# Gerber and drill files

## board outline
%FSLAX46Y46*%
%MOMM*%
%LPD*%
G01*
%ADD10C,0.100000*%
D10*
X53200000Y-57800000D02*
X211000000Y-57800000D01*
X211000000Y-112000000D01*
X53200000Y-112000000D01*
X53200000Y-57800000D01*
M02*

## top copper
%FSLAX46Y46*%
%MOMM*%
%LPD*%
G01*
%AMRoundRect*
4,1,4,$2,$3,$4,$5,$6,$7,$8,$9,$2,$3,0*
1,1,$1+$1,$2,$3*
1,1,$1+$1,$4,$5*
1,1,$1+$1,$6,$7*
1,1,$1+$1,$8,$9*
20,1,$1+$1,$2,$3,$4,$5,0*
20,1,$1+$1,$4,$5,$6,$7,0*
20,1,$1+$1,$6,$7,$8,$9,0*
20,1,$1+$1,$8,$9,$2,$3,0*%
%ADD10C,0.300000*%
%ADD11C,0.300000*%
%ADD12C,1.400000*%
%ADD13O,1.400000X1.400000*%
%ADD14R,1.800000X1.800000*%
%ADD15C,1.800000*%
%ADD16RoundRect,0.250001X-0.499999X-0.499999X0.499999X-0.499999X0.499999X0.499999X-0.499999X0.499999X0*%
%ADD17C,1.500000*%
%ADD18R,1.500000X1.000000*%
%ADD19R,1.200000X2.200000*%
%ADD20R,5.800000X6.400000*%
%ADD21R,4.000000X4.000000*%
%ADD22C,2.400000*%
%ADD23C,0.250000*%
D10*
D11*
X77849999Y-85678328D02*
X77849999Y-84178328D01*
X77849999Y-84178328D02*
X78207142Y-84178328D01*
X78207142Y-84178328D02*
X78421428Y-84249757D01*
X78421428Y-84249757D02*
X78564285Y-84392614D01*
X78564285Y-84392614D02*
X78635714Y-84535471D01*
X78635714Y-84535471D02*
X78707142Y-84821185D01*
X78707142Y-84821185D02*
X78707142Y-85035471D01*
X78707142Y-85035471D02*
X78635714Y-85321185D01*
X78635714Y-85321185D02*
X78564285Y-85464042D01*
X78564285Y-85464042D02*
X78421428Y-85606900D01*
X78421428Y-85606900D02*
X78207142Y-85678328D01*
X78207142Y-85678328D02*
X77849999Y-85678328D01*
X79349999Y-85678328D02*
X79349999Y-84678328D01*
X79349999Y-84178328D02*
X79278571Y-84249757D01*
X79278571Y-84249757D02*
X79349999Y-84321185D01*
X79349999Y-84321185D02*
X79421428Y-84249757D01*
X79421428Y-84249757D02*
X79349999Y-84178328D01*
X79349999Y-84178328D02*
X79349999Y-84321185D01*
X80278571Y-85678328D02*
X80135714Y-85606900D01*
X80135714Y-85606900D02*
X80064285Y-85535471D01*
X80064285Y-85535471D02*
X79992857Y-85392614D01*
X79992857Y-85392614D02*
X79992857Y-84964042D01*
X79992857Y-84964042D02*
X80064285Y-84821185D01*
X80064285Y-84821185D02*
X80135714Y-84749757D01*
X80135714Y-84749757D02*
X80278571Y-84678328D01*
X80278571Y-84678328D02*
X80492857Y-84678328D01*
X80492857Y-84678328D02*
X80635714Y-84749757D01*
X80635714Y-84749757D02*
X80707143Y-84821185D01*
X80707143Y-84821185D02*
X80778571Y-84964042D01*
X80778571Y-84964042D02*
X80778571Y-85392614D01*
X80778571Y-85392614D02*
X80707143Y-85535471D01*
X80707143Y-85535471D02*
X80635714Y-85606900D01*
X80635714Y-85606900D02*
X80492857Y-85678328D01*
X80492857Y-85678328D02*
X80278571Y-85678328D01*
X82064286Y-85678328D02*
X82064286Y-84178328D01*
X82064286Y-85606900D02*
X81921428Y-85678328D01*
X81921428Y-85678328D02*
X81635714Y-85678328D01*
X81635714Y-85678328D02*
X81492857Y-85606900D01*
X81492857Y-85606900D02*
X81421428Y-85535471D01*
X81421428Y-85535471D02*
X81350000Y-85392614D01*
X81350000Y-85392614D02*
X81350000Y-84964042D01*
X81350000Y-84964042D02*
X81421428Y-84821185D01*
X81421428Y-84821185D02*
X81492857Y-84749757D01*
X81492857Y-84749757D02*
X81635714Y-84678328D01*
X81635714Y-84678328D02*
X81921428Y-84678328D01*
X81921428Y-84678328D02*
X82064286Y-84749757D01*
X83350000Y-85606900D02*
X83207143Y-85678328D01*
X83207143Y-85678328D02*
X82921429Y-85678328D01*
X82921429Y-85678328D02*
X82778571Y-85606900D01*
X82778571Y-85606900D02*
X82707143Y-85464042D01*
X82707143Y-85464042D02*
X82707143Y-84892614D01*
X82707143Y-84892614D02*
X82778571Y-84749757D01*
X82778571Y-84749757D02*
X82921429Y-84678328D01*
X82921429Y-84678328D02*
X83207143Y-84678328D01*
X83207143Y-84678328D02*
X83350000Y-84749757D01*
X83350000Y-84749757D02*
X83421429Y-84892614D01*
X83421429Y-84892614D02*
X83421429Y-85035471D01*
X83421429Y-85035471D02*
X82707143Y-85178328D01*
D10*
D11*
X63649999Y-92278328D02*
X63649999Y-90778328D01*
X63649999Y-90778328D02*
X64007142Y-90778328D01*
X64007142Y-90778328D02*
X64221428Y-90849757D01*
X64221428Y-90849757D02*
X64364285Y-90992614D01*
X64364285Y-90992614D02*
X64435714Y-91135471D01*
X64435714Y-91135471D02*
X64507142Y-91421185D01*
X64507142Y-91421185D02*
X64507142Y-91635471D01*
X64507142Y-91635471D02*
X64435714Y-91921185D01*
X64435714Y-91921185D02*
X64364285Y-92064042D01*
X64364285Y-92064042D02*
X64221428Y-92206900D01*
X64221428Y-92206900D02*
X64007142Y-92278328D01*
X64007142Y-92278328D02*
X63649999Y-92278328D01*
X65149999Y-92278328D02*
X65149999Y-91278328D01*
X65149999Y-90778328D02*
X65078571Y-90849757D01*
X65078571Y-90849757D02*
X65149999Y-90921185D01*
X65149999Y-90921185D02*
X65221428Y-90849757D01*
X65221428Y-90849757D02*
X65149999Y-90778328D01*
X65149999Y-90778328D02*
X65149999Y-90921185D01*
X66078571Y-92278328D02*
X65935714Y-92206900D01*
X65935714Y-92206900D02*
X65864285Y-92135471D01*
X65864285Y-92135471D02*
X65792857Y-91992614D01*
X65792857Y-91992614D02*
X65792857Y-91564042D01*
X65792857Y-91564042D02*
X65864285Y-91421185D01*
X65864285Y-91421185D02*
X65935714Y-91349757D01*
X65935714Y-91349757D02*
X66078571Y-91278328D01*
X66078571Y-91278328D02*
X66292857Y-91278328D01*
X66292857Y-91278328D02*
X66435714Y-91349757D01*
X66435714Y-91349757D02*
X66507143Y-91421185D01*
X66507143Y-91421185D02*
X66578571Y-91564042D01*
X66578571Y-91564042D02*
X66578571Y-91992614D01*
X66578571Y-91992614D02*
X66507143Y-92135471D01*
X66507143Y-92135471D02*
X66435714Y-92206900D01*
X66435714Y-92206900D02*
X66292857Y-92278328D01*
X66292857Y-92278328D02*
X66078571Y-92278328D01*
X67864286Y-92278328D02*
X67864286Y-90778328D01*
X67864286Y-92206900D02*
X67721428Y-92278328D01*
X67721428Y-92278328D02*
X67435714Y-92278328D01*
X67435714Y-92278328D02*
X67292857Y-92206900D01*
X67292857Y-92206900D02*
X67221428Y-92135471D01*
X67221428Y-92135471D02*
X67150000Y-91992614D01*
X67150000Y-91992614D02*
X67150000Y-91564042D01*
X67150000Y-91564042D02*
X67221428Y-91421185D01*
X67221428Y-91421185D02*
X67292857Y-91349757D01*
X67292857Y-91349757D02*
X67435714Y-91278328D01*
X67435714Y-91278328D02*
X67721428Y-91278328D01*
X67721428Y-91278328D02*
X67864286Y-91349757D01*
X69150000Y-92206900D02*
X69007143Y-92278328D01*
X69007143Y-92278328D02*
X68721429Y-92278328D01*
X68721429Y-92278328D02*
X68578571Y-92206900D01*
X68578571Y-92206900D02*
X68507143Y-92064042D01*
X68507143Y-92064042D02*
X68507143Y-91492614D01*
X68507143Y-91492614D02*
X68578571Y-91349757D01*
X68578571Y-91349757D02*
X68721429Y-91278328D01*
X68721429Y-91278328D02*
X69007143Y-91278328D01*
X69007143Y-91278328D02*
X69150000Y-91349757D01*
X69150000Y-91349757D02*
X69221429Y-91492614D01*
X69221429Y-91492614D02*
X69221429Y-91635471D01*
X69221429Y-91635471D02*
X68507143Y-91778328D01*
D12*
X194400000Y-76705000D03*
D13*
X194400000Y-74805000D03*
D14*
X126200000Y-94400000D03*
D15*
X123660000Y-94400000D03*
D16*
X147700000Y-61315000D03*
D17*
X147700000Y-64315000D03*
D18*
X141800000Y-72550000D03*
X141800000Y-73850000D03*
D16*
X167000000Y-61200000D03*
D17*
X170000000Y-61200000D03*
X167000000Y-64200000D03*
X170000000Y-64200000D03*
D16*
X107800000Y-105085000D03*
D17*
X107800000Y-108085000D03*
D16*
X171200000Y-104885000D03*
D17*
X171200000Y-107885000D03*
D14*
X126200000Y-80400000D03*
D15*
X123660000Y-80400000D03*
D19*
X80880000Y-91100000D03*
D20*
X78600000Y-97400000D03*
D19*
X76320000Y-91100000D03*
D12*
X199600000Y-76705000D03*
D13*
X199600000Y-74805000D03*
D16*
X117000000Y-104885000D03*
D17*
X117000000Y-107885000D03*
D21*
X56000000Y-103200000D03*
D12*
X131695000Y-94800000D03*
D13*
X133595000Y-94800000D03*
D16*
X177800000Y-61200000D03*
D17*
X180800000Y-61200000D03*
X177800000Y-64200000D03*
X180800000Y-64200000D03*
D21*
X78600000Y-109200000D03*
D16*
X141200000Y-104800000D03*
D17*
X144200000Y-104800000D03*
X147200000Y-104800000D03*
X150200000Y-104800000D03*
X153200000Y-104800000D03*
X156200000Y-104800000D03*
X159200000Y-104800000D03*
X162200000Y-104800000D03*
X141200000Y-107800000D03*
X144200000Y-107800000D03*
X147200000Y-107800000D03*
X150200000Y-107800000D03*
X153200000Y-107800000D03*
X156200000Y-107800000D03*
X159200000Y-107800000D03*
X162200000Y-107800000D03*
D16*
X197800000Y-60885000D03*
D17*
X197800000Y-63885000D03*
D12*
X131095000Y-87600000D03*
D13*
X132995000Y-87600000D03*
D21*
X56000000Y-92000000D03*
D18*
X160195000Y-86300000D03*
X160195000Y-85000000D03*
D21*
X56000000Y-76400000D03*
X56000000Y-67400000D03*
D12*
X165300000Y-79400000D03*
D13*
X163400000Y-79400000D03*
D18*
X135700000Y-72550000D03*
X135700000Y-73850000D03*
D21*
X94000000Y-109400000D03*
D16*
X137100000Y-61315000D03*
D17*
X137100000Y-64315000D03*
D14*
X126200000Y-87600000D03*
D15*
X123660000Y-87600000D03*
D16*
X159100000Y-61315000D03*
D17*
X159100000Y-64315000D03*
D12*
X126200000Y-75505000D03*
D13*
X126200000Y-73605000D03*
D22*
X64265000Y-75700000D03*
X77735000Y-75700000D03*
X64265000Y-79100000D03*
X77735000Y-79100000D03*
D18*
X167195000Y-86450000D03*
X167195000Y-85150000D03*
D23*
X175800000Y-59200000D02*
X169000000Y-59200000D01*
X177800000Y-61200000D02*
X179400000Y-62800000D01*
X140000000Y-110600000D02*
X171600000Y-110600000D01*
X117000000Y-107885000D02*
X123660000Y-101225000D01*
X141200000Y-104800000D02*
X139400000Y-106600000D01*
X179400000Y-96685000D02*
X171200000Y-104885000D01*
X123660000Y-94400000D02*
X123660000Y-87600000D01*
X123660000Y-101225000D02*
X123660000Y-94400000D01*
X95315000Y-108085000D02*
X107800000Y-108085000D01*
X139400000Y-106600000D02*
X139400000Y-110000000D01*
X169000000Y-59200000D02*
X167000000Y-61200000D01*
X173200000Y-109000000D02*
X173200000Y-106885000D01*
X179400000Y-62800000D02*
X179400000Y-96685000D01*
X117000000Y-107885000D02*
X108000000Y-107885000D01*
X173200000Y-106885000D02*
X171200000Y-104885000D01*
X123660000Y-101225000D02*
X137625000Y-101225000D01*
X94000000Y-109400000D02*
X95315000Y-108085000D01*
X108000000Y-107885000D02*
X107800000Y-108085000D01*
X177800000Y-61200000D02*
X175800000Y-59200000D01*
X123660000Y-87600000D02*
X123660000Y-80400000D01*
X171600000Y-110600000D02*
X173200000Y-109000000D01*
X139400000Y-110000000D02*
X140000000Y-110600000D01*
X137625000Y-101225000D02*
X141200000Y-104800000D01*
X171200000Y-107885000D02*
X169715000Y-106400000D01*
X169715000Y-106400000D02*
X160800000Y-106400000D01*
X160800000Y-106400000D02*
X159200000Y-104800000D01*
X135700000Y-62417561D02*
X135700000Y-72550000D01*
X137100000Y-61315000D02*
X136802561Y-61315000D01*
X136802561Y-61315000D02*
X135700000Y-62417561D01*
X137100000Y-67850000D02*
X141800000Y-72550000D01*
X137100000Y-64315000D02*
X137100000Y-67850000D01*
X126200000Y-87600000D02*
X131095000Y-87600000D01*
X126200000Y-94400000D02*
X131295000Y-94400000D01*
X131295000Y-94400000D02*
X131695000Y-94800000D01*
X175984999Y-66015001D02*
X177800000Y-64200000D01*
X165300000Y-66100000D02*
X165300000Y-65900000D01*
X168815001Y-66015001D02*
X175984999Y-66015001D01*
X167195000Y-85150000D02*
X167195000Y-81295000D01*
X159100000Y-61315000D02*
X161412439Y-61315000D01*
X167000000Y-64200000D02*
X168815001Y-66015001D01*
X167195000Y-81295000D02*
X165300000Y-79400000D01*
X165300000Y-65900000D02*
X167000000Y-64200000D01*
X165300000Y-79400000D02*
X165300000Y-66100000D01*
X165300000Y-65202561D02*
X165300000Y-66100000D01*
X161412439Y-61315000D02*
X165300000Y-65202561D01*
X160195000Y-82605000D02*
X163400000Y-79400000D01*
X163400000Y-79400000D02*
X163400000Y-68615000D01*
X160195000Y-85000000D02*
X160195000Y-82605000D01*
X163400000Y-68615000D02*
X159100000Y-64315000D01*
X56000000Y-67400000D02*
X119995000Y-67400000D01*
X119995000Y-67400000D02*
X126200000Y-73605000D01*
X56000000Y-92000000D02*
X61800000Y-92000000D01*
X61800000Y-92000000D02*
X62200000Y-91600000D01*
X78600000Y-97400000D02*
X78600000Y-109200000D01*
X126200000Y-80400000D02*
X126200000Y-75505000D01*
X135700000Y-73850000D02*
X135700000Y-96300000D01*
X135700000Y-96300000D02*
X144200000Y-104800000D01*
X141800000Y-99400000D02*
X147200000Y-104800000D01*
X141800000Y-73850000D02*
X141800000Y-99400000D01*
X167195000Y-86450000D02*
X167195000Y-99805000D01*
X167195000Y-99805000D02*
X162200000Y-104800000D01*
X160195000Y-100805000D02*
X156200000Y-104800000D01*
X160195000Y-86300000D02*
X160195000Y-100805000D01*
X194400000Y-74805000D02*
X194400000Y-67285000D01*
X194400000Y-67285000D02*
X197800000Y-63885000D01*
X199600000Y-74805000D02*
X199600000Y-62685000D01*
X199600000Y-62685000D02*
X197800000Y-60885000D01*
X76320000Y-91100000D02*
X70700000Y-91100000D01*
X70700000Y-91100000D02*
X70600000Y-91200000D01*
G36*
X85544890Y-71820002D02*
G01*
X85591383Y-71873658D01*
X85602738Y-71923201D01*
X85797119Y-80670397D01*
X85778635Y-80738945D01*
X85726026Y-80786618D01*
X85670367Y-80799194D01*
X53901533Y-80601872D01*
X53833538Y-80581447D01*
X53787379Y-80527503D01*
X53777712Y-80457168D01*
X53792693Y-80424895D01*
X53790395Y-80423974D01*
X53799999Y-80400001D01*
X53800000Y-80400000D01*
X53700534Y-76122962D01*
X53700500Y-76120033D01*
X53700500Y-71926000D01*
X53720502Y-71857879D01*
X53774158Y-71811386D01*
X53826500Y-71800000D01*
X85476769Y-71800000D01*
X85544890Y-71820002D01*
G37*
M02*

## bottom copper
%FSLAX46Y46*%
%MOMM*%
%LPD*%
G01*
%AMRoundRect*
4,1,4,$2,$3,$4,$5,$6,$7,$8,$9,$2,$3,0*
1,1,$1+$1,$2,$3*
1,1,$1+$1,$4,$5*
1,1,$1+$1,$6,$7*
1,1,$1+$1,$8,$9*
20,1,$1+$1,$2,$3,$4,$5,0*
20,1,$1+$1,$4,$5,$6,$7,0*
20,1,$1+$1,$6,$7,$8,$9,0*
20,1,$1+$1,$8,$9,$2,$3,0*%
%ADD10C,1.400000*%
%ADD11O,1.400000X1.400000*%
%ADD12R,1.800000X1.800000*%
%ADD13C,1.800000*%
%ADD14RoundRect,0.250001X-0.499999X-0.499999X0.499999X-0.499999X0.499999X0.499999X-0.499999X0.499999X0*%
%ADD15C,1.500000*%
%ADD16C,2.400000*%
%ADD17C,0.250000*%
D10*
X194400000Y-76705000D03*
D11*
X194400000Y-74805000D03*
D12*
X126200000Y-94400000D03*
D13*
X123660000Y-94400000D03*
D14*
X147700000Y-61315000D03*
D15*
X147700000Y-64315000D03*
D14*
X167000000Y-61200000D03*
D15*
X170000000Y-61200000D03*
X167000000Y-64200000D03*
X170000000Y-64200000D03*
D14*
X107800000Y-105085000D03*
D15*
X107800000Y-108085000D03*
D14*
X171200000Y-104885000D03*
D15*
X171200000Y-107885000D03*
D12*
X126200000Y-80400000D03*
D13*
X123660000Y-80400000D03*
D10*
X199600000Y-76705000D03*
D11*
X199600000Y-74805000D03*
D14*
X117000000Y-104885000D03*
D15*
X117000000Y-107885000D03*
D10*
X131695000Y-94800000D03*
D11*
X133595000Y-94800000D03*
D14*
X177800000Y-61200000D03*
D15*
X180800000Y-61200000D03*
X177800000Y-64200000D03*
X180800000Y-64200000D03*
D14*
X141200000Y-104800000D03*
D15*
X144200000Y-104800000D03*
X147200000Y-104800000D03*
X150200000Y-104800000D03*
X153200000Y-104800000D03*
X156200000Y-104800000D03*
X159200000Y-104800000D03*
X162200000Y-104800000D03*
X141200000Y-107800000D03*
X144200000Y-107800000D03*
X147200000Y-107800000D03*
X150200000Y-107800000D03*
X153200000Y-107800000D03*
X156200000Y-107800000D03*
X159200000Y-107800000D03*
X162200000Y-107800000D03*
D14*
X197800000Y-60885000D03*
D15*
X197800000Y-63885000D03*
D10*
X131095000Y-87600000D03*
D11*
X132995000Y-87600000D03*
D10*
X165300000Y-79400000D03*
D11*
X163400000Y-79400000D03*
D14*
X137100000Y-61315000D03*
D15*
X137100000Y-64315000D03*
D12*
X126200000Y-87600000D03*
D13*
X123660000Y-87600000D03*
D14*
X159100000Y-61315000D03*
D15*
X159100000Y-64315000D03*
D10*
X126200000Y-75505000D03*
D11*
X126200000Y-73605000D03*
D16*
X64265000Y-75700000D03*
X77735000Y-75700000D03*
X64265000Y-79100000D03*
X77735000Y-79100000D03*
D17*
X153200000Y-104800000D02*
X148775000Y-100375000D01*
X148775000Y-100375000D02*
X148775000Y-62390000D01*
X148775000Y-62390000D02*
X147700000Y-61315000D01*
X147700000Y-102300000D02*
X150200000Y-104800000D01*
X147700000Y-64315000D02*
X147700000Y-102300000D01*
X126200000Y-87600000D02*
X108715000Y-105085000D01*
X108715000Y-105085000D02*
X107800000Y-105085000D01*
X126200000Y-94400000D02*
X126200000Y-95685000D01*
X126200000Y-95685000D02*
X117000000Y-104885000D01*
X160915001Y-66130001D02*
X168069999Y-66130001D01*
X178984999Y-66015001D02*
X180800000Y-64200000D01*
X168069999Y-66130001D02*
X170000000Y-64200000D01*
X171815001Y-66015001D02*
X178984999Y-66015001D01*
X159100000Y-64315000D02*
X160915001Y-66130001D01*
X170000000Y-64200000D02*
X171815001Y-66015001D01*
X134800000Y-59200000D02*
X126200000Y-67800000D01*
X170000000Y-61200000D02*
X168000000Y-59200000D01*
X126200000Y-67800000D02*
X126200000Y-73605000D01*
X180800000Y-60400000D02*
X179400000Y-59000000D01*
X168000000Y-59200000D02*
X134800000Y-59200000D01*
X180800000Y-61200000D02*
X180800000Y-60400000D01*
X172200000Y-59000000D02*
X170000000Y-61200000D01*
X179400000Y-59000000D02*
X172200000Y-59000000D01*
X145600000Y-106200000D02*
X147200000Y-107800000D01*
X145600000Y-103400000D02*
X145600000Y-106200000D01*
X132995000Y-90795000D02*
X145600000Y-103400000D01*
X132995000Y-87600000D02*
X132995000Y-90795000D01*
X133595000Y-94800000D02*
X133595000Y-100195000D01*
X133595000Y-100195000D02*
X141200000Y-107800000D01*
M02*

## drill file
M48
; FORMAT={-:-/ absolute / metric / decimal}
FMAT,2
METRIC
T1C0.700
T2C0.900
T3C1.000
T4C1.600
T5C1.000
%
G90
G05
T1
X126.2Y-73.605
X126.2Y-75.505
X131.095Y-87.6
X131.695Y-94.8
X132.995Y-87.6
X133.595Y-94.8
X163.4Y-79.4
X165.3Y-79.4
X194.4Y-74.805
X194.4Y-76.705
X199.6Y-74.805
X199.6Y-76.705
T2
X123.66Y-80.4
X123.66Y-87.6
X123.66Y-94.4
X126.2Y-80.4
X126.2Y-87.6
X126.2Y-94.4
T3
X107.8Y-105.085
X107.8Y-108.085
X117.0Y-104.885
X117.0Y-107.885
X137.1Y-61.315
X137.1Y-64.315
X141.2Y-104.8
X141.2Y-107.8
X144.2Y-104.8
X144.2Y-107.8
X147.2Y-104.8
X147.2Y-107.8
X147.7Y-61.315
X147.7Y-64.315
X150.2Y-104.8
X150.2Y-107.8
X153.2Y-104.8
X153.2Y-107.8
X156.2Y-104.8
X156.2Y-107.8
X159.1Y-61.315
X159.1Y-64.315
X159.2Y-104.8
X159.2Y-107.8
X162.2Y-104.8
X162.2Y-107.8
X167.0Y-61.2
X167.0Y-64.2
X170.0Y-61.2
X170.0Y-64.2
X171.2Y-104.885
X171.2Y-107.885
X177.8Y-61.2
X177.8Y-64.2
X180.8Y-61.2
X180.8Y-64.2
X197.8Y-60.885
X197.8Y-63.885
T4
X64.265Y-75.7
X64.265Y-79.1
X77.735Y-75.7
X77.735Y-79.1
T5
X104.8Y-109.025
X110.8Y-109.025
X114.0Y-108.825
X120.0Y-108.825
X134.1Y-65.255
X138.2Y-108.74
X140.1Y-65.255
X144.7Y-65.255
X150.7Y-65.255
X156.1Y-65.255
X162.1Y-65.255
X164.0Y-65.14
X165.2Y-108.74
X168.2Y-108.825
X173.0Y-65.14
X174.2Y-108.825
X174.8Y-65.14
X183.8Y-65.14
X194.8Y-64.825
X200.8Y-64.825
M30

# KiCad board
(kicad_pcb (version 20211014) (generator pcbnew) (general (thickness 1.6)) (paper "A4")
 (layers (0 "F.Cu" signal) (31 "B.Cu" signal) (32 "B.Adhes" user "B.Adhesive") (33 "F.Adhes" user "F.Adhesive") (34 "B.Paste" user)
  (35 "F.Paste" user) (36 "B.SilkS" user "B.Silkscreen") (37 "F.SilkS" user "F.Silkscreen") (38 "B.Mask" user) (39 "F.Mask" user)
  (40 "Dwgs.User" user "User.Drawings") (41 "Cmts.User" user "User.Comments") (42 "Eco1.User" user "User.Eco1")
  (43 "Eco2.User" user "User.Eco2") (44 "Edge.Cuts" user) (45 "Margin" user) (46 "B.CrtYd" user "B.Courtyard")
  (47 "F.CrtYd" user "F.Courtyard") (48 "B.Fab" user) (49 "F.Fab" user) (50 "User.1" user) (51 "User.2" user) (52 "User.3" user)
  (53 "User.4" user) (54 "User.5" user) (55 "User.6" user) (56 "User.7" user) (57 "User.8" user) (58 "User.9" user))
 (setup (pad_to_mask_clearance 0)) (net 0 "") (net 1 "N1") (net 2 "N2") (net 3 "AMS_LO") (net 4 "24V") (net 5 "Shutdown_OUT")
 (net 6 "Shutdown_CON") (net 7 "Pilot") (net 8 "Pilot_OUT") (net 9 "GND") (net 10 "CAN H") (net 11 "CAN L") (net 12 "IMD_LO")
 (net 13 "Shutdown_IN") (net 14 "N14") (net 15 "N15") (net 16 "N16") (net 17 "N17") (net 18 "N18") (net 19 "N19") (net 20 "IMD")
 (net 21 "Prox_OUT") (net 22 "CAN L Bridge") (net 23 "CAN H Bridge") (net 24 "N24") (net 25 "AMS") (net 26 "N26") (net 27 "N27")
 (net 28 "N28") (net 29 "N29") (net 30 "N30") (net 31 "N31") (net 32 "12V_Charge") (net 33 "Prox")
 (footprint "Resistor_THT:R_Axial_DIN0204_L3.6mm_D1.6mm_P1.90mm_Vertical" (layer "F.Cu") (at 194.4 76.705 90)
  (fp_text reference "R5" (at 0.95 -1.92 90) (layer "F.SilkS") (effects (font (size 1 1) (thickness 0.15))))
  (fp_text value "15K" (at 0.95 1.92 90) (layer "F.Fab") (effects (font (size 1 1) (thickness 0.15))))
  (pad "1" thru_hole circle (at 0 0 90) (size 1.4 1.4) (drill 0.7) (layers *.Cu *.Mask) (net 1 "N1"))
  (pad "2" thru_hole oval (at 1.9 0 90) (size 1.4 1.4) (drill 0.7) (layers *.Cu *.Mask) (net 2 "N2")))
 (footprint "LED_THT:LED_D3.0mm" (layer "F.Cu") (at 126.2 94.4 180)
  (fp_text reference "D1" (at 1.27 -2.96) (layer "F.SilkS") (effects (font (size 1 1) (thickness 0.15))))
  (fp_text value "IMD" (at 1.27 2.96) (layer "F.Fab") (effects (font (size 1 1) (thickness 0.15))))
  (pad "1" thru_hole rect (at 0 0 180) (size 1.8 1.8) (drill 0.9) (layers *.Cu *.Mask) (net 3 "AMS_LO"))
  (pad "2" thru_hole circle (at 2.54 0 180) (size 1.8 1.8) (drill 0.9) (layers *.Cu *.Mask) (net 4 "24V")))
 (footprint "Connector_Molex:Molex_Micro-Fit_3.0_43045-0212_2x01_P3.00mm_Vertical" (layer "F.Cu") (at 147.7 61.315)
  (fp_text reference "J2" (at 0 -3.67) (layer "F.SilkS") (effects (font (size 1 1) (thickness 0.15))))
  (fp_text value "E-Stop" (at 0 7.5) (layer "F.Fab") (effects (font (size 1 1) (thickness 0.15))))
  (pad "" np_thru_hole circle (at -3 3.94) (size 1 1) (drill 1) (layers *.Cu *.Mask))
  (pad "" np_thru_hole circle (at 3 3.94) (size 1 1) (drill 1) (layers *.Cu *.Mask))
  (pad "1" thru_hole roundrect (at 0 0) (size 1.5 1.5) (drill 1) (layers *.Cu *.Mask) (roundrect_rratio 0.166667) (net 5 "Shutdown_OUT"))
  (pad "2" thru_hole circle (at 0 3) (size 1.5 1.5) (drill 1) (layers *.Cu *.Mask) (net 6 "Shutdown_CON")))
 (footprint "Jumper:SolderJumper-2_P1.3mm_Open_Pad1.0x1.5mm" (layer "F.Cu") (at 141.8 73.2 -90)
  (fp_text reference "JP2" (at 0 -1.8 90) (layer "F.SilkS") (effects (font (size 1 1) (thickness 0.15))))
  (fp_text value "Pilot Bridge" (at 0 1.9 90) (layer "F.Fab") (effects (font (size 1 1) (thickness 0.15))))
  (pad "1" smd rect (at -0.65 0 270) (size 1 1.5) (layers "F.Cu" "F.Mask") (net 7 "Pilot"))
  (pad "2" smd rect (at 0.65 0 270) (size 1 1.5) (layers "F.Cu" "F.Mask") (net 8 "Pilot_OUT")))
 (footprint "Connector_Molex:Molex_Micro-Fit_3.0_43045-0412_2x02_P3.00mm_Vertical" (layer "F.Cu") (at 167 61.2)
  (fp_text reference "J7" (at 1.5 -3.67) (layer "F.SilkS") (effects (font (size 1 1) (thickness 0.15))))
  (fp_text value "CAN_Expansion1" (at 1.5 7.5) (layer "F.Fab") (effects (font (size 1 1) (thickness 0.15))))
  (pad "" np_thru_hole circle (at -3 3.94) (size 1 1) (drill 1) (layers *.Cu *.Mask))
  (pad "" np_thru_hole circle (at 6 3.94) (size 1 1) (drill 1) (layers *.Cu *.Mask))
  (pad "1" thru_hole roundrect (at 0 0) (size 1.5 1.5) (drill 1) (layers *.Cu *.Mask) (roundrect_rratio 0.166667) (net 4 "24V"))
  (pad "2" thru_hole circle (at 3 0) (size 1.5 1.5) (drill 1) (layers *.Cu *.Mask) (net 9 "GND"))
  (pad "3" thru_hole circle (at 0 3) (size 1.5 1.5) (drill 1) (layers *.Cu *.Mask) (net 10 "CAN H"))
  (pad "4" thru_hole circle (at 3 3) (size 1.5 1.5) (drill 1) (layers *.Cu *.Mask) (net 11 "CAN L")))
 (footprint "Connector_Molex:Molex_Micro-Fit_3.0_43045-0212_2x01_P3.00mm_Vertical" (layer "F.Cu") (at 107.8 105.085)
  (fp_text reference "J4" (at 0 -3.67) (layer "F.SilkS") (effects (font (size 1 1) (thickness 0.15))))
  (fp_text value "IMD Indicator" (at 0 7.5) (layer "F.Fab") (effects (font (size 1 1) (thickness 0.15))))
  (pad "" np_thru_hole circle (at -3 3.94) (size 1 1) (drill 1) (layers *.Cu *.Mask))
  (pad "" np_thru_hole circle (at 3 3.94) (size 1 1) (drill 1) (layers *.Cu *.Mask))
  (pad "1" thru_hole roundrect (at 0 0) (size 1.5 1.5) (drill 1) (layers *.Cu *.Mask) (roundrect_rratio 0.166667) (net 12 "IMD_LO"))
  (pad "2" thru_hole circle (at 0 3) (size 1.5 1.5) (drill 1) (layers *.Cu *.Mask) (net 4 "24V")))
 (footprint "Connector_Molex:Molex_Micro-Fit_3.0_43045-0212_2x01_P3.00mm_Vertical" (layer "F.Cu") (at 171.2 104.885)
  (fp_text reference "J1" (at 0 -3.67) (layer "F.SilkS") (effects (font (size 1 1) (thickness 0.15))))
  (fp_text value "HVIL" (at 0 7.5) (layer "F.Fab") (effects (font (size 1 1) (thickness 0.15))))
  (pad "" np_thru_hole circle (at -3 3.94) (size 1 1) (drill 1) (layers *.Cu *.Mask))
  (pad "" np_thru_hole circle (at 3 3.94) (size 1 1) (drill 1) (layers *.Cu *.Mask))
  (pad "1" thru_hole roundrect (at 0 0) (size 1.5 1.5) (drill 1) (layers *.Cu *.Mask) (roundrect_rratio 0.166667) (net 4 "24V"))
  (pad "2" thru_hole circle (at 0 3) (size 1.5 1.5) (drill 1) (layers *.Cu *.Mask) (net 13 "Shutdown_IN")))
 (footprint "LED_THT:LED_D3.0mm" (layer "F.Cu") (at 126.2 80.4 180)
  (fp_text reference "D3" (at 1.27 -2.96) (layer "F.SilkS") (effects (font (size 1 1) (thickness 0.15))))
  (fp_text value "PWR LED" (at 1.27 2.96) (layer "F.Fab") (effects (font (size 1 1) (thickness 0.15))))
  (pad "1" thru_hole rect (at 0 0 180) (size 1.8 1.8) (drill 0.9) (layers *.Cu *.Mask) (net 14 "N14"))
  (pad "2" thru_hole circle (at 2.54 0 180) (size 1.8 1.8) (drill 0.9) (layers *.Cu *.Mask) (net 4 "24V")))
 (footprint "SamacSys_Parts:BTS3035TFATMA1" (layer "F.Cu") (at 78.6 100.6 180)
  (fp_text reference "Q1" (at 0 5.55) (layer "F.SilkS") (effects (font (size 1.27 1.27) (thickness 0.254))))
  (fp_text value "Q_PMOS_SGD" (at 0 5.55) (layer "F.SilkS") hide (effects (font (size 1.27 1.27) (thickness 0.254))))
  (pad "1" smd rect locked (at -2.28 9.5 180) (size 1.2 2.2) (layers "F.Cu" "F.Paste" "F.Mask") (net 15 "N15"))
  (pad "2" smd rect locked (at 0 3.2 180) (size 5.8 6.4) (layers "F.Cu" "F.Paste" "F.Mask") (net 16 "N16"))
  (pad "3" smd rect locked (at 2.28 9.5 180) (size 1.2 2.2) (layers "F.Cu" "F.Paste" "F.Mask") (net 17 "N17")))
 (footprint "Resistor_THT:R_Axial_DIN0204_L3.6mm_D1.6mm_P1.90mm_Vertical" (layer "F.Cu") (at 199.6 76.705 90)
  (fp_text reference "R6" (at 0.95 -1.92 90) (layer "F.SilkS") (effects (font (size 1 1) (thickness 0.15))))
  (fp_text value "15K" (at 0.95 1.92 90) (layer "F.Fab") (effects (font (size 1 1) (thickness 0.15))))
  (pad "1" thru_hole circle (at 0 0 90) (size 1.4 1.4) (drill 0.7) (layers *.Cu *.Mask) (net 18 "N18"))
  (pad "2" thru_hole oval (at 1.9 0 90) (size 1.4 1.4) (drill 0.7) (layers *.Cu *.Mask) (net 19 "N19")))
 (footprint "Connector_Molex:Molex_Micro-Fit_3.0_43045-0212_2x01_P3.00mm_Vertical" (layer "F.Cu") (at 117 104.885)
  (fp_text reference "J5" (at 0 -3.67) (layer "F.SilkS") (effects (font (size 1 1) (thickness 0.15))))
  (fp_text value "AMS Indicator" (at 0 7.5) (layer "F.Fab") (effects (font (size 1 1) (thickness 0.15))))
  (pad "" np_thru_hole circle (at 3 3.94) (size 1 1) (drill 1) (layers *.Cu *.Mask))
  (pad "" np_thru_hole circle (at -3 3.94) (size 1 1) (drill 1) (layers *.Cu *.Mask))
  (pad "1" thru_hole roundrect (at 0 0) (size 1.5 1.5) (drill 1) (layers *.Cu *.Mask) (roundrect_rratio 0.166667) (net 3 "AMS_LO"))
  (pad "2" thru_hole circle (at 0 3) (size 1.5 1.5) (drill 1) (layers *.Cu *.Mask) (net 4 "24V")))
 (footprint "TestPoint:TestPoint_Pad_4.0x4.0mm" (layer "F.Cu") (at 56 103.2)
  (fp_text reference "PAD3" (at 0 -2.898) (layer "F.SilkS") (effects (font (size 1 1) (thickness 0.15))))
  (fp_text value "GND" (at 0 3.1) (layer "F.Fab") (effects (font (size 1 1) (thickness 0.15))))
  (pad "1" smd rect (at 0 0) (size 4 4) (layers "F.Cu" "F.Mask") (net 9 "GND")))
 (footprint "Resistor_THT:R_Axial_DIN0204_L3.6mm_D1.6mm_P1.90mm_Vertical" (layer "F.Cu") (at 131.695 94.8)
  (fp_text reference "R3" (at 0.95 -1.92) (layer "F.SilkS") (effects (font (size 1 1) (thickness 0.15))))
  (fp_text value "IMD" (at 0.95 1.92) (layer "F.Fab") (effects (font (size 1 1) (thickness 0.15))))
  (pad "1" thru_hole circle (at 0 0) (size 1.4 1.4) (drill 0.7) (layers *.Cu *.Mask) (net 3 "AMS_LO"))
  (pad "2" thru_hole oval (at 1.9 0) (size 1.4 1.4) (drill 0.7) (layers *.Cu *.Mask) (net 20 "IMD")))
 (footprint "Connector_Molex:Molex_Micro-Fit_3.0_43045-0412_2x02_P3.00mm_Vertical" (layer "F.Cu") (at 177.8 61.2)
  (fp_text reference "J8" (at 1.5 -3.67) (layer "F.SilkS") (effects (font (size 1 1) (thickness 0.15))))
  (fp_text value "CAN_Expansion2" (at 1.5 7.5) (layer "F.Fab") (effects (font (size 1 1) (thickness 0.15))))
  (pad "" np_thru_hole circle (at 6 3.94) (size 1 1) (drill 1) (layers *.Cu *.Mask))
  (pad "" np_thru_hole circle (at -3 3.94) (size 1 1) (drill 1) (layers *.Cu *.Mask))
  (pad "1" thru_hole roundrect (at 0 0) (size 1.5 1.5) (drill 1) (layers *.Cu *.Mask) (roundrect_rratio 0.166667) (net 4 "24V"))
  (pad "2" thru_hole circle (at 3 0) (size 1.5 1.5) (drill 1) (layers *.Cu *.Mask) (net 9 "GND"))
  (pad "3" thru_hole circle (at 0 3) (size 1.5 1.5) (drill 1) (layers *.Cu *.Mask) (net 10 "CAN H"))
  (pad "4" thru_hole circle (at 3 3) (size 1.5 1.5) (drill 1) (layers *.Cu *.Mask) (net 11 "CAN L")))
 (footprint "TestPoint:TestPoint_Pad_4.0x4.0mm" (layer "F.Cu") (at 78.6 109.2)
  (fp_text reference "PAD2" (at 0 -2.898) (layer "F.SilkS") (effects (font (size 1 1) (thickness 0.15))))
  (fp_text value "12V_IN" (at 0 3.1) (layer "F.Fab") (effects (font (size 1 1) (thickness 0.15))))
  (pad "1" smd rect (at 0 0) (size 4 4) (layers "F.Cu" "F.Mask") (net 16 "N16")))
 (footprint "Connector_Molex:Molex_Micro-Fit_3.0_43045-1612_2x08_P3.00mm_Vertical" (layer "F.Cu") (at 141.2 104.8)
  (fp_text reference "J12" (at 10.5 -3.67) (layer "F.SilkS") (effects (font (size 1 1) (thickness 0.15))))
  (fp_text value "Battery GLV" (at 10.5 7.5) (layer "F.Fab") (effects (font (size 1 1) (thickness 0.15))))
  (pad "" np_thru_hole circle (at -3 3.94) (size 1 1) (drill 1) (layers *.Cu *.Mask))
  (pad "" np_thru_hole circle (at 24 3.94) (size 1 1) (drill 1) (layers *.Cu *.Mask))
  (pad "1" thru_hole roundrect (at 0 0) (size 1.5 1.5) (drill 1) (layers *.Cu *.Mask) (roundrect_rratio 0.166667) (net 4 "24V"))
  (pad "2" thru_hole circle (at 3 0) (size 1.5 1.5) (drill 1) (layers *.Cu *.Mask) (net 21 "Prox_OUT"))
  (pad "3" thru_hole circle (at 6 0) (size 1.5 1.5) (drill 1) (layers *.Cu *.Mask) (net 8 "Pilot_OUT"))
  (pad "4" thru_hole circle (at 9 0) (size 1.5 1.5) (drill 1) (layers *.Cu *.Mask) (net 6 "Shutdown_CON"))
  (pad "5" thru_hole circle (at 12 0) (size 1.5 1.5) (drill 1) (layers *.Cu *.Mask) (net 5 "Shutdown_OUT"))
  (pad "6" thru_hole circle (at 15 0) (size 1.5 1.5) (drill 1) (layers *.Cu *.Mask) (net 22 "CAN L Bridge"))
  (pad "7" thru_hole circle (at 18 0) (size 1.5 1.5) (drill 1) (layers *.Cu *.Mask) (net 13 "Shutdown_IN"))
  (pad "8" thru_hole circle (at 21 0) (size 1.5 1.5) (drill 1) (layers *.Cu *.Mask) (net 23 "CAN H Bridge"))
  (pad "9" thru_hole circle (at 0 3) (size 1.5 1.5) (drill 1) (layers *.Cu *.Mask) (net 20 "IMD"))
  (pad "10" thru_hole circle (at 3 3) (size 1.5 1.5) (drill 1) (layers *.Cu *.Mask) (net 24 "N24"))
  (pad "11" thru_hole circle (at 6 3) (size 1.5 1.5) (drill 1) (layers *.Cu *.Mask) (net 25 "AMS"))
  (pad "12" thru_hole circle (at 9 3) (size 1.5 1.5) (drill 1) (layers *.Cu *.Mask) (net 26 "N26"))
  (pad "13" thru_hole circle (at 12 3) (size 1.5 1.5) (drill 1) (layers *.Cu *.Mask) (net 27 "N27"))
  (pad "14" thru_hole circle (at 15 3) (size 1.5 1.5) (drill 1) (layers *.Cu *.Mask) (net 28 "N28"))
  (pad "15" thru_hole circle (at 18 3) (size 1.5 1.5) (drill 1) (layers *.Cu *.Mask) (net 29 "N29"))
  (pad "16" thru_hole circle (at 21 3) (size 1.5 1.5) (drill 1) (layers *.Cu *.Mask) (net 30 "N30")))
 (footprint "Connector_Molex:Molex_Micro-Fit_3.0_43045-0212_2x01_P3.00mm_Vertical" (layer "F.Cu") (at 197.8 60.885)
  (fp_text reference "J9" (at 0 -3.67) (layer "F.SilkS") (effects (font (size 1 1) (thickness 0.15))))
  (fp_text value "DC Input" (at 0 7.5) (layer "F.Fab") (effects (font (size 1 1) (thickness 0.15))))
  (pad "" np_thru_hole circle (at -3 3.94) (size 1 1) (drill 1) (layers *.Cu *.Mask))
  (pad "" np_thru_hole circle (at 3 3.94) (size 1 1) (drill 1) (layers *.Cu *.Mask))
  (pad "1" thru_hole roundrect (at 0 0) (size 1.5 1.5) (drill 1) (layers *.Cu *.Mask) (roundrect_rratio 0.166667) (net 19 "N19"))
  (pad "2" thru_hole circle (at 0 3) (size 1.5 1.5) (drill 1) (layers *.Cu *.Mask) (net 2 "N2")))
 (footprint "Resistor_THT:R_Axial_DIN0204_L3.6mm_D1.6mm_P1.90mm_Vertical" (layer "F.Cu") (at 131.095 87.6)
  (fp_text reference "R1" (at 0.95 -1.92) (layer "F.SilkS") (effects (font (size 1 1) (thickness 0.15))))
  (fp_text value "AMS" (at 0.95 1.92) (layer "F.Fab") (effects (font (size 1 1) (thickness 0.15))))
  (pad "1" thru_hole circle (at 0 0) (size 1.4 1.4) (drill 0.7) (layers *.Cu *.Mask) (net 12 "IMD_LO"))
  (pad "2" thru_hole oval (at 1.9 0) (size 1.4 1.4) (drill 0.7) (layers *.Cu *.Mask) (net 25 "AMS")))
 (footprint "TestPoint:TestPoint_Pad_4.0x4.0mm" (layer "F.Cu") (at 56 92)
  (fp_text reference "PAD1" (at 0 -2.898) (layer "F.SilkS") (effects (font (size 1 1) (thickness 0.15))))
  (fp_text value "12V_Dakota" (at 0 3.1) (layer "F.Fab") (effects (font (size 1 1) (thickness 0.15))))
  (pad "1" smd rect (at 0 0) (size 4 4) (layers "F.Cu" "F.Mask") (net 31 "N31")))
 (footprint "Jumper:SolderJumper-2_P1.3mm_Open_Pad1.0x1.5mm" (layer "F.Cu") (at 160.195 85.65 90)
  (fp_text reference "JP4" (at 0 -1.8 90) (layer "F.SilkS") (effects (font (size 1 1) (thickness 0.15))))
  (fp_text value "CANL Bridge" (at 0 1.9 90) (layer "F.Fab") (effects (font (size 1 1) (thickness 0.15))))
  (pad "1" smd rect (at -0.65 0 90) (size 1 1.5) (layers "F.Cu" "F.Mask") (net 22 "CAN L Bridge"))
  (pad "2" smd rect (at 0.65 0 90) (size 1 1.5) (layers "F.Cu" "F.Mask") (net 11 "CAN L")))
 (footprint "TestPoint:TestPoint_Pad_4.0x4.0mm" (layer "F.Cu") (at 56 76.4)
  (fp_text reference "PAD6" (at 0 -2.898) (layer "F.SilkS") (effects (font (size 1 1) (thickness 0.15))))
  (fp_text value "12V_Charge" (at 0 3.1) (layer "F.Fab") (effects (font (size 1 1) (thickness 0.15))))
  (pad "1" smd rect (at 0 0) (size 4 4) (layers "F.Cu" "F.Mask") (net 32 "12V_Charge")))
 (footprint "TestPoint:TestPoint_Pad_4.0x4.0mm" (layer "F.Cu") (at 56 67.4)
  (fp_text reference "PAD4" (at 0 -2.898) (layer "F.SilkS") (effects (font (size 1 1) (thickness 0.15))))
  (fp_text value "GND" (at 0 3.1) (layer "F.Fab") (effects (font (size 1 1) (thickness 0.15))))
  (pad "1" smd rect (at 0 0) (size 4 4) (layers "F.Cu" "F.Mask") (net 9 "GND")))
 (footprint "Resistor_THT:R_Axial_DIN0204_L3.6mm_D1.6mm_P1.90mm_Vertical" (layer "F.Cu") (at 165.3 79.4 180)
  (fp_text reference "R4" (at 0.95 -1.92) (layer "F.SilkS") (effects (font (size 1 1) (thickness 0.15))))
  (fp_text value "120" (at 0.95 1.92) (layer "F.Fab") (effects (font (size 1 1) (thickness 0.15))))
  (pad "1" thru_hole circle (at 0 0 180) (size 1.4 1.4) (drill 0.7) (layers *.Cu *.Mask) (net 10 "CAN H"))
  (pad "2" thru_hole oval (at 1.9 0 180) (size 1.4 1.4) (drill 0.7) (layers *.Cu *.Mask) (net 11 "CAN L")))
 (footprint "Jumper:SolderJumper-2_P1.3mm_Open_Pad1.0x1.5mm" (layer "F.Cu") (at 135.7 73.2 -90)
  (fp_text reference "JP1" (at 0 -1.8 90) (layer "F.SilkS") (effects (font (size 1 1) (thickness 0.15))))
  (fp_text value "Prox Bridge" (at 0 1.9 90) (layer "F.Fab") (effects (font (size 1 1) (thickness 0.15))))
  (pad "1" smd rect (at -0.65 0 270) (size 1 1.5) (layers "F.Cu" "F.Mask") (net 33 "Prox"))
  (pad "2" smd rect (at 0.65 0 270) (size 1 1.5) (layers "F.Cu" "F.Mask") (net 21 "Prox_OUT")))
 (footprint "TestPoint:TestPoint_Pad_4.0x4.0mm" (layer "F.Cu") (at 94 109.4)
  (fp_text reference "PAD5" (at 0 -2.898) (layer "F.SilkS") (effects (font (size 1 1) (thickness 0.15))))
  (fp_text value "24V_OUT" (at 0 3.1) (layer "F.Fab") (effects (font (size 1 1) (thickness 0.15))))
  (pad "1" smd rect (at 0 0) (size 4 4) (layers "F.Cu" "F.Mask") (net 4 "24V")))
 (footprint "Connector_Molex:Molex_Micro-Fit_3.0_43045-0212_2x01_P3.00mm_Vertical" (layer "F.Cu") (at 137.1 61.315)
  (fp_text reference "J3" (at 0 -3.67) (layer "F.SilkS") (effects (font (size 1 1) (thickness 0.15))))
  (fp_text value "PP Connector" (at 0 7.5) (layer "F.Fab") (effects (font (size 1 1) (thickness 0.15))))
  (pad "" np_thru_hole circle (at 3 3.94) (size 1 1) (drill 1) (layers *.Cu *.Mask))
  (pad "" np_thru_hole circle (at -3 3.94) (size 1 1) (drill 1) (layers *.Cu *.Mask))
  (pad "1" thru_hole roundrect (at 0 0) (size 1.5 1.5) (drill 1) (layers *.Cu *.Mask) (roundrect_rratio 0.166667) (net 33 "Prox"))
  (pad "2" thru_hole circle (at 0 3) (size 1.5 1.5) (drill 1) (layers *.Cu *.Mask) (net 7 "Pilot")))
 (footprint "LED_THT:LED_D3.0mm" (layer "F.Cu") (at 126.2 87.6 180)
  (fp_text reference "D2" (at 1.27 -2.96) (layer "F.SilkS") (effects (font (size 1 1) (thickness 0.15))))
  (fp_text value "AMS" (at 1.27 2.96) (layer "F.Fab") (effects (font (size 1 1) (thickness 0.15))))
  (pad "1" thru_hole rect (at 0 0 180) (size 1.8 1.8) (drill 0.9) (layers *.Cu *.Mask) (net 12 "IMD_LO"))
  (pad "2" thru_hole circle (at 2.54 0 180) (size 1.8 1.8) (drill 0.9) (layers *.Cu *.Mask) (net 4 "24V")))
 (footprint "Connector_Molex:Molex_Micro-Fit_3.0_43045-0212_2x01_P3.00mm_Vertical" (layer "F.Cu") (at 159.1 61.315)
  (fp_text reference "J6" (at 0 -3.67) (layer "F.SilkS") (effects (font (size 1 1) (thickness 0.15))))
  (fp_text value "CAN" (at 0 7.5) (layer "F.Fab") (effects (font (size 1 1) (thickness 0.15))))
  (pad "" np_thru_hole circle (at -3 3.94) (size 1 1) (drill 1) (layers *.Cu *.Mask))
  (pad "" np_thru_hole circle (at 3 3.94) (size 1 1) (drill 1) (layers *.Cu *.Mask))
  (pad "1" thru_hole roundrect (at 0 0) (size 1.5 1.5) (drill 1) (layers *.Cu *.Mask) (roundrect_rratio 0.166667) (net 10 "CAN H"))
  (pad "2" thru_hole circle (at 0 3) (size 1.5 1.5) (drill 1) (layers *.Cu *.Mask) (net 11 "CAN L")))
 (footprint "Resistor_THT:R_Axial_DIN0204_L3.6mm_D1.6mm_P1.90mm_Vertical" (layer "F.Cu") (at 126.2 75.505 90)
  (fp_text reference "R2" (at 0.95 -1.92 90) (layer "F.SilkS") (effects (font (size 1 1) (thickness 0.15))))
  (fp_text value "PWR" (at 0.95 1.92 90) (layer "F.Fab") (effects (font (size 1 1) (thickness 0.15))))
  (pad "1" thru_hole circle (at 0 0 90) (size 1.4 1.4) (drill 0.7) (layers *.Cu *.Mask) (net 14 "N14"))
  (pad "2" thru_hole oval (at 1.9 0 90) (size 1.4 1.4) (drill 0.7) (layers *.Cu *.Mask) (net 9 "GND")))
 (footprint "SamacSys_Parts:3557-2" (layer "F.Cu") (at 71 77.4)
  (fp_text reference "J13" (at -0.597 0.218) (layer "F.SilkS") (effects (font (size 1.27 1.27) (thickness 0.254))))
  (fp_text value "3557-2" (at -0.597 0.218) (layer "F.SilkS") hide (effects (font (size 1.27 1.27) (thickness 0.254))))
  (pad "1" thru_hole circle locked (at -6.735 -1.7) (size 2.4 2.4) (drill 1.6) (layers *.Cu *.Mask) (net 32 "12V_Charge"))
  (pad "2" thru_hole circle locked (at 6.735 -1.7) (size 2.4 2.4) (drill 1.6) (layers *.Cu *.Mask) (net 32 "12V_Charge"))
  (pad "3" thru_hole circle locked (at -6.735 1.7) (size 2.4 2.4) (drill 1.6) (layers *.Cu *.Mask) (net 32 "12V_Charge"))
  (pad "4" thru_hole circle locked (at 6.735 1.7) (size 2.4 2.4) (drill 1.6) (layers *.Cu *.Mask) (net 32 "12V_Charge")))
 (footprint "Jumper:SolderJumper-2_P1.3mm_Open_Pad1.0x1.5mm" (layer "F.Cu") (at 167.195 85.8 90)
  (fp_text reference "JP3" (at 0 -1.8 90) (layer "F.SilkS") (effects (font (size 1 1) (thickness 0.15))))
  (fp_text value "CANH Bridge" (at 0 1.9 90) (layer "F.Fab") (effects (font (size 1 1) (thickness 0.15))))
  (pad "1" smd rect (at -0.65 0 90) (size 1 1.5) (layers "F.Cu" "F.Mask") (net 23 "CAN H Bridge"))
  (pad "2" smd rect (at 0.65 0 90) (size 1 1.5) (layers "F.Cu" "F.Mask") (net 10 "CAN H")))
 (gr_rect (start 53.2 57.8) (end 211 112) (layer "Edge.Cuts") (width 0.1) (fill none))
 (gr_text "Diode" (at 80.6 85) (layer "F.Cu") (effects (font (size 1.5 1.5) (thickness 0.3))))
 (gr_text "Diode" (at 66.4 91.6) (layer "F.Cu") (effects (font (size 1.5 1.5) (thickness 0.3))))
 (segment (start 175.8 59.2) (end 169 59.2) (width 0.25) (layer "F.Cu") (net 4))
 (segment (start 177.8 61.2) (end 179.4 62.8) (width 0.25) (layer "F.Cu") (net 4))
 (segment (start 140 110.6) (end 171.6 110.6) (width 0.25) (layer "F.Cu") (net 4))
 (segment (start 117 107.885) (end 123.66 101.225) (width 0.25) (layer "F.Cu") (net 4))
 (segment (start 141.2 104.8) (end 139.4 106.6) (width 0.25) (layer "F.Cu") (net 4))
 (segment (start 179.4 96.685) (end 171.2 104.885) (width 0.25) (layer "F.Cu") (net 4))
 (segment (start 123.66 94.4) (end 123.66 87.6) (width 0.25) (layer "F.Cu") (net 4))
 (segment (start 123.66 101.225) (end 123.66 94.4) (width 0.25) (layer "F.Cu") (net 4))
 (segment (start 95.315 108.085) (end 107.8 108.085) (width 0.25) (layer "F.Cu") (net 4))
 (segment (start 139.4 106.6) (end 139.4 110) (width 0.25) (layer "F.Cu") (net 4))
 (segment (start 169 59.2) (end 167 61.2) (width 0.25) (layer "F.Cu") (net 4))
 (segment (start 173.2 109) (end 173.2 106.885) (width 0.25) (layer "F.Cu") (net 4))
 (segment (start 179.4 62.8) (end 179.4 96.685) (width 0.25) (layer "F.Cu") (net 4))
 (segment (start 117 107.885) (end 108 107.885) (width 0.25) (layer "F.Cu") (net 4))
 (segment (start 173.2 106.885) (end 171.2 104.885) (width 0.25) (layer "F.Cu") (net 4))
 (segment (start 123.66 101.225) (end 137.625 101.225) (width 0.25) (layer "F.Cu") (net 4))
 (segment (start 94 109.4) (end 95.315 108.085) (width 0.25) (layer "F.Cu") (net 4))
 (segment (start 108 107.885) (end 107.8 108.085) (width 0.25) (layer "F.Cu") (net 4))
 (segment (start 177.8 61.2) (end 175.8 59.2) (width 0.25) (layer "F.Cu") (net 4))
 (segment (start 123.66 87.6) (end 123.66 80.4) (width 0.25) (layer "F.Cu") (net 4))
 (segment (start 171.6 110.6) (end 173.2 109) (width 0.25) (layer "F.Cu") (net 4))
 (segment (start 139.4 110) (end 140 110.6) (width 0.25) (layer "F.Cu") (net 4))
 (segment (start 137.625 101.225) (end 141.2 104.8) (width 0.25) (layer "F.Cu") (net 4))
 (segment (start 171.2 107.885) (end 169.715 106.4) (width 0.25) (layer "F.Cu") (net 13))
 (segment (start 169.715 106.4) (end 160.8 106.4) (width 0.25) (layer "F.Cu") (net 13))
 (segment (start 160.8 106.4) (end 159.2 104.8) (width 0.25) (layer "F.Cu") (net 13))
 (segment (start 153.2 104.8) (end 148.775 100.375) (width 0.25) (layer "B.Cu") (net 5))
 (segment (start 148.775 100.375) (end 148.775 62.39) (width 0.25) (layer "B.Cu") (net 5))
 (segment (start 148.775 62.39) (end 147.7 61.315) (width 0.25) (layer "B.Cu") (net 5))
 (segment (start 147.7 102.3) (end 150.2 104.8) (width 0.25) (layer "B.Cu") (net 6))
 (segment (start 147.7 64.315) (end 147.7 102.3) (width 0.25) (layer "B.Cu") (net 6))
 (segment (start 135.7 62.417561) (end 135.7 72.55) (width 0.25) (layer "F.Cu") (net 33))
 (segment (start 137.1 61.315) (end 136.802561 61.315) (width 0.25) (layer "F.Cu") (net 33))
 (segment (start 136.802561 61.315) (end 135.7 62.417561) (width 0.25) (layer "F.Cu") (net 33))
 (segment (start 137.1 67.85) (end 141.8 72.55) (width 0.25) (layer "F.Cu") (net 7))
 (segment (start 137.1 64.315) (end 137.1 67.85) (width 0.25) (layer "F.Cu") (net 7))
 (segment (start 126.2 87.6) (end 131.095 87.6) (width 0.25) (layer "F.Cu") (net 12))
 (segment (start 126.2 87.6) (end 108.715 105.085) (width 0.25) (layer "B.Cu") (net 12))
 (segment (start 108.715 105.085) (end 107.8 105.085) (width 0.25) (layer "B.Cu") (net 12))
 (segment (start 126.2 94.4) (end 131.295 94.4) (width 0.25) (layer "F.Cu") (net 3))
 (segment (start 131.295 94.4) (end 131.695 94.8) (width 0.25) (layer "F.Cu") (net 3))
 (segment (start 126.2 94.4) (end 126.2 95.685) (width 0.25) (layer "B.Cu") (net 3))
 (segment (start 126.2 95.685) (end 117 104.885) (width 0.25) (layer "B.Cu") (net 3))
 (segment (start 175.984999 66.015001) (end 177.8 64.2) (width 0.25) (layer "F.Cu") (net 10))
 (segment (start 165.3 66.1) (end 165.3 65.9) (width 0.25) (layer "F.Cu") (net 10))
 (segment (start 168.815001 66.015001) (end 175.984999 66.015001) (width 0.25) (layer "F.Cu") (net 10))
 (segment (start 167.195 85.15) (end 167.195 81.295) (width 0.25) (layer "F.Cu") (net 10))
 (segment (start 159.1 61.315) (end 161.412439 61.315) (width 0.25) (layer "F.Cu") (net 10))
 (segment (start 167 64.2) (end 168.815001 66.015001) (width 0.25) (layer "F.Cu") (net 10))
 (segment (start 167.195 81.295) (end 165.3 79.4) (width 0.25) (layer "F.Cu") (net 10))
 (segment (start 165.3 65.9) (end 167 64.2) (width 0.25) (layer "F.Cu") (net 10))
 (segment (start 165.3 79.4) (end 165.3 66.1) (width 0.25) (layer "F.Cu") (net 10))
 (segment (start 165.3 65.202561) (end 165.3 66.1) (width 0.25) (layer "F.Cu") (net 10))
 (segment (start 161.412439 61.315) (end 165.3 65.202561) (width 0.25) (layer "F.Cu") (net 10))
 (segment (start 160.195 82.605) (end 163.4 79.4) (width 0.25) (layer "F.Cu") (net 11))
 (segment (start 163.4 79.4) (end 163.4 68.615) (width 0.25) (layer "F.Cu") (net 11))
 (segment (start 160.195 85) (end 160.195 82.605) (width 0.25) (layer "F.Cu") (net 11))
 (segment (start 163.4 68.615) (end 159.1 64.315) (width 0.25) (layer "F.Cu") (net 11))
 (segment (start 160.915001 66.130001) (end 168.069999 66.130001) (width 0.25) (layer "B.Cu") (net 11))
 (segment (start 178.984999 66.015001) (end 180.8 64.2) (width 0.25) (layer "B.Cu") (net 11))
 (segment (start 168.069999 66.130001) (end 170 64.2) (width 0.25) (layer "B.Cu") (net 11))
 (segment (start 171.815001 66.015001) (end 178.984999 66.015001) (width 0.25) (layer "B.Cu") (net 11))
 (segment (start 159.1 64.315) (end 160.915001 66.130001) (width 0.25) (layer "B.Cu") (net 11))
 (segment (start 170 64.2) (end 171.815001 66.015001) (width 0.25) (layer "B.Cu") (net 11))
 (segment (start 56 67.4) (end 119.995 67.4) (width 0.25) (layer "F.Cu") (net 9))
 (segment (start 119.995 67.4) (end 126.2 73.605) (width 0.25) (layer "F.Cu") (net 9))
 (segment (start 134.8 59.2) (end 126.2 67.8) (width 0.25) (layer "B.Cu") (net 9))
 (segment (start 170 61.2) (end 168 59.2) (width 0.25) (layer "B.Cu") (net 9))
 (segment (start 126.2 67.8) (end 126.2 73.605) (width 0.25) (layer "B.Cu") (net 9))
 (segment (start 180.8 60.4) (end 179.4 59) (width 0.25) (layer "B.Cu") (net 9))
 (segment (start 168 59.2) (end 134.8 59.2) (width 0.25) (layer "B.Cu") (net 9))
 (segment (start 180.8 61.2) (end 180.8 60.4) (width 0.25) (layer "B.Cu") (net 9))
 (segment (start 172.2 59) (end 170 61.2) (width 0.25) (layer "B.Cu") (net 9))
 (segment (start 179.4 59) (end 172.2 59) (width 0.25) (layer "B.Cu") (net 9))
 (segment (start 56 92) (end 61.8 92) (width 0.25) (layer "F.Cu") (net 31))
 (segment (start 61.8 92) (end 62.2 91.6) (width 0.25) (layer "F.Cu") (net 31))
 (segment (start 78.6 97.4) (end 78.6 109.2) (width 0.25) (layer "F.Cu") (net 16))
 (segment (start 126.2 80.4) (end 126.2 75.505) (width 0.25) (layer "F.Cu") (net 14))
 (segment (start 135.7 73.85) (end 135.7 96.3) (width 0.25) (layer "F.Cu") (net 21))
 (segment (start 135.7 96.3) (end 144.2 104.8) (width 0.25) (layer "F.Cu") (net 21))
 (segment (start 141.8 99.4) (end 147.2 104.8) (width 0.25) (layer "F.Cu") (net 8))
 (segment (start 141.8 73.85) (end 141.8 99.4) (width 0.25) (layer "F.Cu") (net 8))
 (segment (start 167.195 86.45) (end 167.195 99.805) (width 0.25) (layer "F.Cu") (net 23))
 (segment (start 167.195 99.805) (end 162.2 104.8) (width 0.25) (layer "F.Cu") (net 23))
 (segment (start 160.195 100.805) (end 156.2 104.8) (width 0.25) (layer "F.Cu") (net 22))
 (segment (start 160.195 86.3) (end 160.195 100.805) (width 0.25) (layer "F.Cu") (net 22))
 (segment (start 145.6 106.2) (end 147.2 107.8) (width 0.25) (layer "B.Cu") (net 25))
 (segment (start 145.6 103.4) (end 145.6 106.2) (width 0.25) (layer "B.Cu") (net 25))
 (segment (start 132.995 90.795) (end 145.6 103.4) (width 0.25) (layer "B.Cu") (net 25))
 (segment (start 132.995 87.6) (end 132.995 90.795) (width 0.25) (layer "B.Cu") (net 25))
 (segment (start 133.595 94.8) (end 133.595 100.195) (width 0.25) (layer "B.Cu") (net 20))
 (segment (start 133.595 100.195) (end 141.2 107.8) (width 0.25) (layer "B.Cu") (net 20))
 (segment (start 194.4 74.805) (end 194.4 67.285) (width 0.25) (layer "F.Cu") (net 2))
 (segment (start 194.4 67.285) (end 197.8 63.885) (width 0.25) (layer "F.Cu") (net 2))
 (segment (start 199.6 74.805) (end 199.6 62.685) (width 0.25) (layer "F.Cu") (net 19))
 (segment (start 199.6 62.685) (end 197.8 60.885) (width 0.25) (layer "F.Cu") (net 19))
 (segment (start 76.32 91.1) (end 70.7 91.1) (width 0.25) (layer "F.Cu") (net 17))
 (segment (start 70.7 91.1) (end 70.6 91.2) (width 0.25) (layer "F.Cu") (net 17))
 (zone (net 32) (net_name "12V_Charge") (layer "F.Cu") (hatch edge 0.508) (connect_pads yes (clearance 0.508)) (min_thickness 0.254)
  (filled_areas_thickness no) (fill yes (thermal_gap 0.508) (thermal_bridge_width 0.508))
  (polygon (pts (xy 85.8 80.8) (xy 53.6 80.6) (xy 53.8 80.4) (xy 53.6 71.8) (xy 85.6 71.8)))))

